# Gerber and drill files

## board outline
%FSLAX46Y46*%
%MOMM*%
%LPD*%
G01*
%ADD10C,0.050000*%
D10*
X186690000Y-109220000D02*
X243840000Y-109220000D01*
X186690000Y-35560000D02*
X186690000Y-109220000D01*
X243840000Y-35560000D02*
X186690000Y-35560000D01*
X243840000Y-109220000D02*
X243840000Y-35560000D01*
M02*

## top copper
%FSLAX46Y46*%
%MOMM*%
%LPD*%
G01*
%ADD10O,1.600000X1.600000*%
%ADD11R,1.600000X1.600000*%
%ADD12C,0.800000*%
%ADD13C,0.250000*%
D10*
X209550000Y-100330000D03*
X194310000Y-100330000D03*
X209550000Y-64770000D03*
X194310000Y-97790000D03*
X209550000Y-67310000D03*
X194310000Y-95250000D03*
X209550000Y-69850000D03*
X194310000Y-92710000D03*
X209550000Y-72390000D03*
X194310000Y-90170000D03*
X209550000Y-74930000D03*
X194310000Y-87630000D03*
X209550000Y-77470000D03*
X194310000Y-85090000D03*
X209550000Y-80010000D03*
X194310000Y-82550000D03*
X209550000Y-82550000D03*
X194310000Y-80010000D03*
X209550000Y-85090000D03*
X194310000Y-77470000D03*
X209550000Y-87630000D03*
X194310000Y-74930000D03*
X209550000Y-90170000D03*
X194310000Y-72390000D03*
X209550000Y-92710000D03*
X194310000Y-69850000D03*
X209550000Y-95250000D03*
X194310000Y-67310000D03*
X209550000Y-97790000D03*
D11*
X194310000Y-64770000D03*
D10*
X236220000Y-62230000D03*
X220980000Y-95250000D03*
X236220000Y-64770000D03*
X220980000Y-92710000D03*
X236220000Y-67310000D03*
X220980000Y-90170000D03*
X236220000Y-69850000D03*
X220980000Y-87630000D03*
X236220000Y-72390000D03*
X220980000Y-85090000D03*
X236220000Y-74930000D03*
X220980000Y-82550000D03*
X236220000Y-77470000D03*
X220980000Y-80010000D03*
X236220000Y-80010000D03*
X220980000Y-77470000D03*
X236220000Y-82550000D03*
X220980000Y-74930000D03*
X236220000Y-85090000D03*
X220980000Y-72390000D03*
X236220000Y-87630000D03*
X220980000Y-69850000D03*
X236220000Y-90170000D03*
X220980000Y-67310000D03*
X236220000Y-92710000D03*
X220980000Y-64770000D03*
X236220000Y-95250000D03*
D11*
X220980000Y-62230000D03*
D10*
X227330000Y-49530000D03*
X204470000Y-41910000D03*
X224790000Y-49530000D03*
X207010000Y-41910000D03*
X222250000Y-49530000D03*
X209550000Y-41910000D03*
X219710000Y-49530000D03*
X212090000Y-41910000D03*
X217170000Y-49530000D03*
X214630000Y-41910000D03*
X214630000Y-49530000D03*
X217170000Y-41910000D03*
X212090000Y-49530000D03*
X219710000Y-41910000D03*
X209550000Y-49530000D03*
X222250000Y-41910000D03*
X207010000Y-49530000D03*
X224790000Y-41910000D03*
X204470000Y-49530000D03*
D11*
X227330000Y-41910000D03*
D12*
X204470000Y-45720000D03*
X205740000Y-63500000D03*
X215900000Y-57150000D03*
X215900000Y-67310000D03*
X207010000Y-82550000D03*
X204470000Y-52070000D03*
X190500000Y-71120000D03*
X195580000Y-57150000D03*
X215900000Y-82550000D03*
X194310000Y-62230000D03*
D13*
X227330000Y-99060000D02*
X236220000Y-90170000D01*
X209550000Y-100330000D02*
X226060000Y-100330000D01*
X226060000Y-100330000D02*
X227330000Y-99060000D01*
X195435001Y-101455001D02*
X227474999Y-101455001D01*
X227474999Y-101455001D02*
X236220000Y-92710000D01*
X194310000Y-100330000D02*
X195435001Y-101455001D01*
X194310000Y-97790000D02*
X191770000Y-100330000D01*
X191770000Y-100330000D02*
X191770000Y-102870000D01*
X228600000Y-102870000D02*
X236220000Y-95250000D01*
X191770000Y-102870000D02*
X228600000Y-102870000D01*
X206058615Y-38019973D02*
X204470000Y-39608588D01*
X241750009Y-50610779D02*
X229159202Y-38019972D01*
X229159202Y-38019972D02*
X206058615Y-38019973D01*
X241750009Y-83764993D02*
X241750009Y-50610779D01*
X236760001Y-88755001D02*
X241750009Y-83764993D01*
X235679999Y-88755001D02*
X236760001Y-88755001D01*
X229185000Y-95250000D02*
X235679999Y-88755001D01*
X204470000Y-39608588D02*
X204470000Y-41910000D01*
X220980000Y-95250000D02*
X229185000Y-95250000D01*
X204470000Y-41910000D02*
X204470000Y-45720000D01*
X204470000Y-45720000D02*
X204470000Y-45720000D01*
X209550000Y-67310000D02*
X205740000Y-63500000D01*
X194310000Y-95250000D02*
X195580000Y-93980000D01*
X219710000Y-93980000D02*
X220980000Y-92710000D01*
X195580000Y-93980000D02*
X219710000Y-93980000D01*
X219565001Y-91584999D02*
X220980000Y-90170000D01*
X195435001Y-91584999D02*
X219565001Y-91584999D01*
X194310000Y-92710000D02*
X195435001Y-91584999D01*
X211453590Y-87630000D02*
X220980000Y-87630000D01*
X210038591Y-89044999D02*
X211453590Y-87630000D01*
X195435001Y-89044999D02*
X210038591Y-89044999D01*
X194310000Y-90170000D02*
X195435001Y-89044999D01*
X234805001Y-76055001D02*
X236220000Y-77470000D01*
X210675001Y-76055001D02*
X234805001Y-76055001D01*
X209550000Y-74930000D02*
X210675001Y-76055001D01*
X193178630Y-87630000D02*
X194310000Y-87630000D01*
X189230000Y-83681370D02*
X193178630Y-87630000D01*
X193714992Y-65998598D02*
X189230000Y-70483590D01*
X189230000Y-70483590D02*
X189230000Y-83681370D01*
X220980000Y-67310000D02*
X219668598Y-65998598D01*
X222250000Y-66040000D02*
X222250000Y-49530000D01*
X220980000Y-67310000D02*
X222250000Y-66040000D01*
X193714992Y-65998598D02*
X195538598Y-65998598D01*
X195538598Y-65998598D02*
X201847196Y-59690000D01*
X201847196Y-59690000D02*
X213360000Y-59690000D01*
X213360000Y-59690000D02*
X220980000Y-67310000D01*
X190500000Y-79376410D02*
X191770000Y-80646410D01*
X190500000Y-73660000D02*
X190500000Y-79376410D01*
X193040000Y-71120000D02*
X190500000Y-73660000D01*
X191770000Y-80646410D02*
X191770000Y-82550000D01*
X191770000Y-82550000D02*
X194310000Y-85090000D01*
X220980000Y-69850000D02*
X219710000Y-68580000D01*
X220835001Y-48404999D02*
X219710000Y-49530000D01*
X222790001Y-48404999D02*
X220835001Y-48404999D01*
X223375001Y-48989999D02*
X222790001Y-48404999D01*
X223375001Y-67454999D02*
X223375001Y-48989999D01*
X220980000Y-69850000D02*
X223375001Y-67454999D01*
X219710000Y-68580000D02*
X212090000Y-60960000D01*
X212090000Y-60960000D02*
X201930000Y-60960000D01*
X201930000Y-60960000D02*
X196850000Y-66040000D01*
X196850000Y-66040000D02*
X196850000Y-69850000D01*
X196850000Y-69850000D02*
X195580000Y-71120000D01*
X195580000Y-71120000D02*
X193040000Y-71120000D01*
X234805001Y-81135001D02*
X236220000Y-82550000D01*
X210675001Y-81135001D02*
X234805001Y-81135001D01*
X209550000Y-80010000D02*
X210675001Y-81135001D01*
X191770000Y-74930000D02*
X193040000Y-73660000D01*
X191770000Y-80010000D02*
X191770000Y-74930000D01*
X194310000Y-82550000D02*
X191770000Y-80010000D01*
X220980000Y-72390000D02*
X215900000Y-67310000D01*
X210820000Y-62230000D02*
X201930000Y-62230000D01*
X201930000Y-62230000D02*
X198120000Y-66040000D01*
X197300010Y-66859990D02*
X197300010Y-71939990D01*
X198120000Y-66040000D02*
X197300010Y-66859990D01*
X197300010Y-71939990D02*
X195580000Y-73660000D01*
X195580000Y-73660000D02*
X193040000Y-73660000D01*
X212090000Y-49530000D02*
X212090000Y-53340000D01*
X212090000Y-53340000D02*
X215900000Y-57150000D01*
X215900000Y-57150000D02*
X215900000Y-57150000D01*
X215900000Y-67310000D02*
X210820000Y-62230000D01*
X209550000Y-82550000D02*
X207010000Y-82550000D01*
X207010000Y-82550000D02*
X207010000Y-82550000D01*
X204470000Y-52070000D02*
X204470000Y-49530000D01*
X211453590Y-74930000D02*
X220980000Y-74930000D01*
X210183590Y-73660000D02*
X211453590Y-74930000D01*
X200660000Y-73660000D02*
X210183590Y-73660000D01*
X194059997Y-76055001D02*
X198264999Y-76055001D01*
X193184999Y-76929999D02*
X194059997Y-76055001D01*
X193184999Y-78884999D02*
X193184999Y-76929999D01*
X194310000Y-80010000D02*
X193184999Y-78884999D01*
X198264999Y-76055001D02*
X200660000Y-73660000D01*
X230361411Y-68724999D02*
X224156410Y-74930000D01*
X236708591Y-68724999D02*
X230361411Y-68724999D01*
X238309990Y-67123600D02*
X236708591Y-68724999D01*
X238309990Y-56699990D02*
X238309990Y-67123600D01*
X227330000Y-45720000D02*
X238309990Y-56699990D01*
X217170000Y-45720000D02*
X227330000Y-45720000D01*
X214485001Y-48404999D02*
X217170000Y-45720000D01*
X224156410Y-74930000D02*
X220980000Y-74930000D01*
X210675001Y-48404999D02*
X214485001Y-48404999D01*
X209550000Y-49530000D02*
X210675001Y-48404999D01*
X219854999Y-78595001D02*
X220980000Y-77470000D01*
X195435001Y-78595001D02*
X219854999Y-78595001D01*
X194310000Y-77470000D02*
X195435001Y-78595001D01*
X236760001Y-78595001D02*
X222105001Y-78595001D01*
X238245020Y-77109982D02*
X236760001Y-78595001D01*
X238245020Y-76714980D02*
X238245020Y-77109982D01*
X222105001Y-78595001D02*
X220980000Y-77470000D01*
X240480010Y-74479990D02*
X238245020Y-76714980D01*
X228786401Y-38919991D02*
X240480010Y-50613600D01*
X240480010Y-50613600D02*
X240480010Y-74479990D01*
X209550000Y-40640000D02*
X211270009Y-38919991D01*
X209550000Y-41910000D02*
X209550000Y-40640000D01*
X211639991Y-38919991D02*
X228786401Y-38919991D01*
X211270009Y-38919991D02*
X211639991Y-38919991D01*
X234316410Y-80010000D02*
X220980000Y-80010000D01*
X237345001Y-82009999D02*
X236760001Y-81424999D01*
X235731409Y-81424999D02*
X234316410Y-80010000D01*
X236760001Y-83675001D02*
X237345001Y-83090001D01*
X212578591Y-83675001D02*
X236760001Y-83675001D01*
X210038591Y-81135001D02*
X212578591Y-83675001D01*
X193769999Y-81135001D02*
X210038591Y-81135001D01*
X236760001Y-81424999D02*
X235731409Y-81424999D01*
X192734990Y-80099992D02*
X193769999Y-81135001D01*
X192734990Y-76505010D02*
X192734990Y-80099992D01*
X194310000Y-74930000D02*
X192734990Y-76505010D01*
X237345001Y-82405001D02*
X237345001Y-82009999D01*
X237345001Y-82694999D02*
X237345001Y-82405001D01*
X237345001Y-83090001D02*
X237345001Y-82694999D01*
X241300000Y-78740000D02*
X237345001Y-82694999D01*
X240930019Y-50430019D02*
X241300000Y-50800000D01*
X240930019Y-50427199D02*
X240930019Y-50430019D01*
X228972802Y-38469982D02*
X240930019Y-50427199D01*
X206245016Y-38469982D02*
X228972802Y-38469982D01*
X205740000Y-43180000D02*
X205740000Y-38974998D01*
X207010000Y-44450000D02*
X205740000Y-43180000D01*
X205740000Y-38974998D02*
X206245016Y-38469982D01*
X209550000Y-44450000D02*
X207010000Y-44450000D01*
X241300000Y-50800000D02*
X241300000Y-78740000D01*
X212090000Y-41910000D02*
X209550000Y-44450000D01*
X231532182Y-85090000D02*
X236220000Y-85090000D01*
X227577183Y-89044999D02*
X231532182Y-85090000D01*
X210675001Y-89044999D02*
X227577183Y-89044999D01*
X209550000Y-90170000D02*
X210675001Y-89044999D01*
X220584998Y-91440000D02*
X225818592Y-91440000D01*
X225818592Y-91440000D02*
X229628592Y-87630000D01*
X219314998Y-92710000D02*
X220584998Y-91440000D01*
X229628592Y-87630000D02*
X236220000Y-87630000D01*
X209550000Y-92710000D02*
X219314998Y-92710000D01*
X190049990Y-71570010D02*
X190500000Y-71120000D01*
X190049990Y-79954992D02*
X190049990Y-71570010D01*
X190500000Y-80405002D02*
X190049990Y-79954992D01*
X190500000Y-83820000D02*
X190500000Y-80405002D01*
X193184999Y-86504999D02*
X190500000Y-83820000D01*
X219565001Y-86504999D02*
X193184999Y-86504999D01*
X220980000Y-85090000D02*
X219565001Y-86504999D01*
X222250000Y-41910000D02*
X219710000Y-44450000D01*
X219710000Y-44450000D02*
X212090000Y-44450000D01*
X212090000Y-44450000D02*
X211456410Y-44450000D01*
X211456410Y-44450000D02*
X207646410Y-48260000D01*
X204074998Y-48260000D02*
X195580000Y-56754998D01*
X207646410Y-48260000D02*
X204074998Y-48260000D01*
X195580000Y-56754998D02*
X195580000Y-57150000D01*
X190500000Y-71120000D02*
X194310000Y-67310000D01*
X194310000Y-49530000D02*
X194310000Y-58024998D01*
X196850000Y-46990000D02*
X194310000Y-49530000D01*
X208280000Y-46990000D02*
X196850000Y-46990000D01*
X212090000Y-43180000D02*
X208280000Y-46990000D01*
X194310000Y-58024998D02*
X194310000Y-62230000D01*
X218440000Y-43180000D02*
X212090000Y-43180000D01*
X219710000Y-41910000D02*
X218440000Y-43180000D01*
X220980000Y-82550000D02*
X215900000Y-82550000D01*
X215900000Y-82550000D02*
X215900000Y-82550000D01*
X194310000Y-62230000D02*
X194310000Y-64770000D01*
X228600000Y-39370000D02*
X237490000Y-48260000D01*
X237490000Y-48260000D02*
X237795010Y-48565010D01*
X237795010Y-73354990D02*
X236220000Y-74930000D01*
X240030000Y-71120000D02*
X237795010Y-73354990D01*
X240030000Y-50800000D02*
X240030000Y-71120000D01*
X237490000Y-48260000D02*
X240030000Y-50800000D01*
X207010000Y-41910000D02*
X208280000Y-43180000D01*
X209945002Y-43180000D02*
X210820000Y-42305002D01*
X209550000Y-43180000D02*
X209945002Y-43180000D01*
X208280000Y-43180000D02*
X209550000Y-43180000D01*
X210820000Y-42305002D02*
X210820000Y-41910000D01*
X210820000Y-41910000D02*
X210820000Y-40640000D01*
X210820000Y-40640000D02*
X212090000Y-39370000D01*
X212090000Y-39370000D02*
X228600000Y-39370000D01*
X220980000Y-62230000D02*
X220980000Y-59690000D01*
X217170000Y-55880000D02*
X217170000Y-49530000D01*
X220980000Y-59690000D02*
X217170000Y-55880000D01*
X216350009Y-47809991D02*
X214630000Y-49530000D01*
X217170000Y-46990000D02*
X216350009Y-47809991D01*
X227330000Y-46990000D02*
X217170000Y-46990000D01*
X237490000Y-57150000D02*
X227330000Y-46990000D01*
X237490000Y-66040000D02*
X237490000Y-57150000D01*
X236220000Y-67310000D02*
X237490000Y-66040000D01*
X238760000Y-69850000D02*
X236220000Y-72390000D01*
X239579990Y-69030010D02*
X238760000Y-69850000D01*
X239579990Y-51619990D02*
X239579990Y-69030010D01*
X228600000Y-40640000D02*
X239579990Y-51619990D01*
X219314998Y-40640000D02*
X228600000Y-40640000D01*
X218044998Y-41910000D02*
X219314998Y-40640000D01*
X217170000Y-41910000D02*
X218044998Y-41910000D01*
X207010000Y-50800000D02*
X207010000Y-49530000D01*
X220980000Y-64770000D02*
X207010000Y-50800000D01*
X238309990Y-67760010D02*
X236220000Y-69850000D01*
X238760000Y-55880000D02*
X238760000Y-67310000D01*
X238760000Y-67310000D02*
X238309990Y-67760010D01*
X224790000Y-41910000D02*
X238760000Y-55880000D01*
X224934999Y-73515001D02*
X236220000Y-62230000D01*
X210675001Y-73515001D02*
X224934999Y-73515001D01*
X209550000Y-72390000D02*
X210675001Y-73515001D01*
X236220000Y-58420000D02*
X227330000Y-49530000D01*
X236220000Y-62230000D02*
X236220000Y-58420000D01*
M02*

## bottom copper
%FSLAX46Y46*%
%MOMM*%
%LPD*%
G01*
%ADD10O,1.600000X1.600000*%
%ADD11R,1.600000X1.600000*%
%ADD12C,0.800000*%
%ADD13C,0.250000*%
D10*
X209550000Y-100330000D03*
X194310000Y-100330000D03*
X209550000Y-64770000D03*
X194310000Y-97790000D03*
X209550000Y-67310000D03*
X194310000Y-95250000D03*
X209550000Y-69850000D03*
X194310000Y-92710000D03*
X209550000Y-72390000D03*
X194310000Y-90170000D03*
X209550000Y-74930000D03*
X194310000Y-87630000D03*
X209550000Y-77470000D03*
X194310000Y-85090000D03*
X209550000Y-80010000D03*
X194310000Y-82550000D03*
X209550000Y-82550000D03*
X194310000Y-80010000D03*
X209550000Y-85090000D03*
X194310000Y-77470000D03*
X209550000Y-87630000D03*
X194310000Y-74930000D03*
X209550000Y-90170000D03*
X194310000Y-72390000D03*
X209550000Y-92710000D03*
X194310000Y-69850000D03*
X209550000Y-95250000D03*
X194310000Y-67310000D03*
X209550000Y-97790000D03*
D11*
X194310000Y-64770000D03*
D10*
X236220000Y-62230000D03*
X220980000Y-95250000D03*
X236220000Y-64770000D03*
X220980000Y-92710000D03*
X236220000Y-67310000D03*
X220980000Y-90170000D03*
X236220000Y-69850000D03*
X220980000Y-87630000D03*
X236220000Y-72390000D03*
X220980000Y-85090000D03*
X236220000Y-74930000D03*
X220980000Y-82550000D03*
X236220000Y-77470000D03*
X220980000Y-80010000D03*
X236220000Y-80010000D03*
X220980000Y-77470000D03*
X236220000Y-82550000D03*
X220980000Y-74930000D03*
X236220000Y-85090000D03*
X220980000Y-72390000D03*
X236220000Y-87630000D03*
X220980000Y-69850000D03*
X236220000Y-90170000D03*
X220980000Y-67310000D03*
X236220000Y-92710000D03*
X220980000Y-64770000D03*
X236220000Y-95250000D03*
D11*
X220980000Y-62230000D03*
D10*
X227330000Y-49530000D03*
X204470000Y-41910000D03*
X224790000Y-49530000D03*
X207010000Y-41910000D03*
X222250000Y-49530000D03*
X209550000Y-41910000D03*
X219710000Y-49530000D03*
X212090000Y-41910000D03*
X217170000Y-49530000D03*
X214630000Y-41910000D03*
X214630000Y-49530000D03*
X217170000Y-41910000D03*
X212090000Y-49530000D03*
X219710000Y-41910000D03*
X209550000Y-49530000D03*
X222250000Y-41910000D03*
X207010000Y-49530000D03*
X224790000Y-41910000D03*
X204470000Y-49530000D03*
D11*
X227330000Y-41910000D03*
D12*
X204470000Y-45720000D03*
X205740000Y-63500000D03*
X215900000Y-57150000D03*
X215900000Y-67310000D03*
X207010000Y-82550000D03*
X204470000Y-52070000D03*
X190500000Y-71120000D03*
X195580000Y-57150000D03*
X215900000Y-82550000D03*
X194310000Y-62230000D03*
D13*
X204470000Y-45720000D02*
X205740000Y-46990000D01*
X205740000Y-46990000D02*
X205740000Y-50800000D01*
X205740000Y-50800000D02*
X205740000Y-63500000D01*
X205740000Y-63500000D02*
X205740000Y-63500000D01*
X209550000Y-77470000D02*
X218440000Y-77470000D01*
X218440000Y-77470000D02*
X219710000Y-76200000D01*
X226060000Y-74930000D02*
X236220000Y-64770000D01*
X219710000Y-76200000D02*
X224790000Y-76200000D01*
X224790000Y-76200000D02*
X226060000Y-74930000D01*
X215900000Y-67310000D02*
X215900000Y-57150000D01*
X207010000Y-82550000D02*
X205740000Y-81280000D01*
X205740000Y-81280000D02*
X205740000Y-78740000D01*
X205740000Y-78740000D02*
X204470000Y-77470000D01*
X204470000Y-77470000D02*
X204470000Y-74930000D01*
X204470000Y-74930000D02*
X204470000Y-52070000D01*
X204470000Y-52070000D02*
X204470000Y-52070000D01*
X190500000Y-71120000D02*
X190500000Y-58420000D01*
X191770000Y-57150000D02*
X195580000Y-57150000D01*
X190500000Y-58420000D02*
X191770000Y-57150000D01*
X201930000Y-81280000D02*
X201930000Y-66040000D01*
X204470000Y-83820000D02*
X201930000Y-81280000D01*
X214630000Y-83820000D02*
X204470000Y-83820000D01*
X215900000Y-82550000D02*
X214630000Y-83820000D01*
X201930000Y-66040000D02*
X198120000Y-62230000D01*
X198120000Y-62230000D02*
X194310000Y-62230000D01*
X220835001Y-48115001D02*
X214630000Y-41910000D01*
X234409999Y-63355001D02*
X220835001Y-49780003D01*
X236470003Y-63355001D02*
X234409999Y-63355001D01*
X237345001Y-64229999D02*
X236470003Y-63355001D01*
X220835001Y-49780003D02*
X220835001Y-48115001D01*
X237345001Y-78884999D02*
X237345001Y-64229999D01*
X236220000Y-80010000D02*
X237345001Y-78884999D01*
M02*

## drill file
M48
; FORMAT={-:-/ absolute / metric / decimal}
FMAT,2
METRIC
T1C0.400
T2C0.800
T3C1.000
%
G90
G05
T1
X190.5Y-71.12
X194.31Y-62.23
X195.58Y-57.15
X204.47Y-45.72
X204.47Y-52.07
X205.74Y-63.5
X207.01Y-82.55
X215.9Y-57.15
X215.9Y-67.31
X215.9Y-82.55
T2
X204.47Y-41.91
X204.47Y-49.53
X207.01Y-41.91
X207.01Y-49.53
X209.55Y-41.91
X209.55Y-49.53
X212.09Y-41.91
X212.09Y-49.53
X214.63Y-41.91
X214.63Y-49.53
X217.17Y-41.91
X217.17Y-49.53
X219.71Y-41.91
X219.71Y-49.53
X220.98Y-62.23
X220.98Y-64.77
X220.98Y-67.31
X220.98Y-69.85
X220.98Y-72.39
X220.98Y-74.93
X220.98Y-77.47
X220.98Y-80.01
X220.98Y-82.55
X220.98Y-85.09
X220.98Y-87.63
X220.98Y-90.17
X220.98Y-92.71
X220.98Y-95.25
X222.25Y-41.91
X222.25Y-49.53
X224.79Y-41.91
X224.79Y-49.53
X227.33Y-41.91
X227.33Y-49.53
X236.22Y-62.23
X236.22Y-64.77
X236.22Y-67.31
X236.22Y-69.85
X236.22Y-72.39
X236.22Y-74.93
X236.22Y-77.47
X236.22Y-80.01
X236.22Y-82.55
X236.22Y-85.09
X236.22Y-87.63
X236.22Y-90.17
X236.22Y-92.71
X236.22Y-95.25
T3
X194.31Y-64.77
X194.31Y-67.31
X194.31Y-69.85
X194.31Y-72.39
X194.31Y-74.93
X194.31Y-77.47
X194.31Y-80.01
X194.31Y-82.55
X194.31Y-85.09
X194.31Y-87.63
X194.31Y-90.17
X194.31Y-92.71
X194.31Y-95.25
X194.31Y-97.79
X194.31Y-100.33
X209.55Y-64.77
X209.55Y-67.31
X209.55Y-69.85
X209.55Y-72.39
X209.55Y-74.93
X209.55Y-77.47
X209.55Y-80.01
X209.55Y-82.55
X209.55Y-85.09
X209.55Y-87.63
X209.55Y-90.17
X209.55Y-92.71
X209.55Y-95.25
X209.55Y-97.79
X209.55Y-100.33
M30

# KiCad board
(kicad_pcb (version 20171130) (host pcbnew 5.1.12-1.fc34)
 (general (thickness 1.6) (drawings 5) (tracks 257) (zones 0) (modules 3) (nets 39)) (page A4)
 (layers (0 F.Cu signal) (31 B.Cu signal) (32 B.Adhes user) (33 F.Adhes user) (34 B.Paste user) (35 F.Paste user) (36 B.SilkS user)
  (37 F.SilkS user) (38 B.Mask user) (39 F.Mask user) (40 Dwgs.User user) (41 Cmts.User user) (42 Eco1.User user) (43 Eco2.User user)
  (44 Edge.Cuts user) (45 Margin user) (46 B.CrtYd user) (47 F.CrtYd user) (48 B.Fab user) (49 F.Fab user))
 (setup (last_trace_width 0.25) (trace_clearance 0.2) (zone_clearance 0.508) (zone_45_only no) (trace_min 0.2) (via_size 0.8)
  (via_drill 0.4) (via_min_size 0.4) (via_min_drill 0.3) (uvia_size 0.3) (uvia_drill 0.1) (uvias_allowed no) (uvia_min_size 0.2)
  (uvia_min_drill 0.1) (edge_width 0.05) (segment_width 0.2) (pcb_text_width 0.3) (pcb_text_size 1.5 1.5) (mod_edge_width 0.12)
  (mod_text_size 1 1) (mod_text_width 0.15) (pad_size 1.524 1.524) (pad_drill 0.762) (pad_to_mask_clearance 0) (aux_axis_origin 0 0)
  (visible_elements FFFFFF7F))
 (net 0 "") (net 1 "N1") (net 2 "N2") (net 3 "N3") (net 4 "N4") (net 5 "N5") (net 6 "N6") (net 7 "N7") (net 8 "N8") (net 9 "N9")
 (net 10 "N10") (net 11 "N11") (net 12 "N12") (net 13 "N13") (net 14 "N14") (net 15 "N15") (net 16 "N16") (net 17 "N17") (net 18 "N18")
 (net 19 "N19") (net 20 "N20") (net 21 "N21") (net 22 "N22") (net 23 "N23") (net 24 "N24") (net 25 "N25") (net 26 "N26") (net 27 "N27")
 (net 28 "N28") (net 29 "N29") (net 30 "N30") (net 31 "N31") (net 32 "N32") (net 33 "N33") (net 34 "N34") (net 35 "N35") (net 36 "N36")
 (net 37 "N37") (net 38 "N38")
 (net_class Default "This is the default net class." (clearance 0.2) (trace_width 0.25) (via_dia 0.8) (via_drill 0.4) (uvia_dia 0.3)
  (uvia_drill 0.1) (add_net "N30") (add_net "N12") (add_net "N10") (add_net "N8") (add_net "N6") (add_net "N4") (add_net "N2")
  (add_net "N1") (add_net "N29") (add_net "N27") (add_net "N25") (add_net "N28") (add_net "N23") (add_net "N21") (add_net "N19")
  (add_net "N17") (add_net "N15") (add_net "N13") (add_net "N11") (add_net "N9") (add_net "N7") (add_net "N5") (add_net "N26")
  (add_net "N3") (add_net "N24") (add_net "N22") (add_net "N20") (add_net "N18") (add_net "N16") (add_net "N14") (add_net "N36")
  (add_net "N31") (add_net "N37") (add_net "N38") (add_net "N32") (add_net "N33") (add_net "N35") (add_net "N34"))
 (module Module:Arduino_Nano (layer F.Cu) (at 194.31 64.77)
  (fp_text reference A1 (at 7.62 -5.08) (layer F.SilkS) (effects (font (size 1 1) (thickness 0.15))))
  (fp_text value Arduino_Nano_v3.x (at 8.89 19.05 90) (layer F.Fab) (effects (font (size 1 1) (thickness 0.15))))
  (pad 16 thru_hole oval (at 15.24 35.56) (size 1.6 1.6) (drill 1) (layers *.Cu *.Mask) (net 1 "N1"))
  (pad 15 thru_hole oval (at 0 35.56) (size 1.6 1.6) (drill 1) (layers *.Cu *.Mask) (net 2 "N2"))
  (pad 30 thru_hole oval (at 15.24 0) (size 1.6 1.6) (drill 1) (layers *.Cu *.Mask) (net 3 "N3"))
  (pad 14 thru_hole oval (at 0 33.02) (size 1.6 1.6) (drill 1) (layers *.Cu *.Mask) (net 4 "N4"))
  (pad 29 thru_hole oval (at 15.24 2.54) (size 1.6 1.6) (drill 1) (layers *.Cu *.Mask) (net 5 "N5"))
  (pad 13 thru_hole oval (at 0 30.48) (size 1.6 1.6) (drill 1) (layers *.Cu *.Mask) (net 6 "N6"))
  (pad 28 thru_hole oval (at 15.24 5.08) (size 1.6 1.6) (drill 1) (layers *.Cu *.Mask) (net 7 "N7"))
  (pad 12 thru_hole oval (at 0 27.94) (size 1.6 1.6) (drill 1) (layers *.Cu *.Mask) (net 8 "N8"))
  (pad 27 thru_hole oval (at 15.24 7.62) (size 1.6 1.6) (drill 1) (layers *.Cu *.Mask) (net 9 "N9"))
  (pad 11 thru_hole oval (at 0 25.4) (size 1.6 1.6) (drill 1) (layers *.Cu *.Mask) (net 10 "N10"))
  (pad 26 thru_hole oval (at 15.24 10.16) (size 1.6 1.6) (drill 1) (layers *.Cu *.Mask) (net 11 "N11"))
  (pad 10 thru_hole oval (at 0 22.86) (size 1.6 1.6) (drill 1) (layers *.Cu *.Mask) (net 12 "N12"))
  (pad 25 thru_hole oval (at 15.24 12.7) (size 1.6 1.6) (drill 1) (layers *.Cu *.Mask) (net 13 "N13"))
  (pad 9 thru_hole oval (at 0 20.32) (size 1.6 1.6) (drill 1) (layers *.Cu *.Mask) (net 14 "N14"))
  (pad 24 thru_hole oval (at 15.24 15.24) (size 1.6 1.6) (drill 1) (layers *.Cu *.Mask) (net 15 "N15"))
  (pad 8 thru_hole oval (at 0 17.78) (size 1.6 1.6) (drill 1) (layers *.Cu *.Mask) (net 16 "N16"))
  (pad 23 thru_hole oval (at 15.24 17.78) (size 1.6 1.6) (drill 1) (layers *.Cu *.Mask) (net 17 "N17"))
  (pad 7 thru_hole oval (at 0 15.24) (size 1.6 1.6) (drill 1) (layers *.Cu *.Mask) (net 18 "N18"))
  (pad 22 thru_hole oval (at 15.24 20.32) (size 1.6 1.6) (drill 1) (layers *.Cu *.Mask) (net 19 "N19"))
  (pad 6 thru_hole oval (at 0 12.7) (size 1.6 1.6) (drill 1) (layers *.Cu *.Mask) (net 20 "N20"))
  (pad 21 thru_hole oval (at 15.24 22.86) (size 1.6 1.6) (drill 1) (layers *.Cu *.Mask) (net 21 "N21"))
  (pad 5 thru_hole oval (at 0 10.16) (size 1.6 1.6) (drill 1) (layers *.Cu *.Mask) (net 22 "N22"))
  (pad 20 thru_hole oval (at 15.24 25.4) (size 1.6 1.6) (drill 1) (layers *.Cu *.Mask) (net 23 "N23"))
  (pad 4 thru_hole oval (at 0 7.62) (size 1.6 1.6) (drill 1) (layers *.Cu *.Mask) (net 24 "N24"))
  (pad 19 thru_hole oval (at 15.24 27.94) (size 1.6 1.6) (drill 1) (layers *.Cu *.Mask) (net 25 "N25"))
  (pad 3 thru_hole oval (at 0 5.08) (size 1.6 1.6) (drill 1) (layers *.Cu *.Mask) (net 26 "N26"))
  (pad 18 thru_hole oval (at 15.24 30.48) (size 1.6 1.6) (drill 1) (layers *.Cu *.Mask) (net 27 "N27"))
  (pad 2 thru_hole oval (at 0 2.54) (size 1.6 1.6) (drill 1) (layers *.Cu *.Mask) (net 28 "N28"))
  (pad 17 thru_hole oval (at 15.24 33.02) (size 1.6 1.6) (drill 1) (layers *.Cu *.Mask) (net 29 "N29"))
  (pad 1 thru_hole rect (at 0 0) (size 1.6 1.6) (drill 1) (layers *.Cu *.Mask) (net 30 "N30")))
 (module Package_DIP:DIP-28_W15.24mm (layer F.Cu) (at 220.98 62.23)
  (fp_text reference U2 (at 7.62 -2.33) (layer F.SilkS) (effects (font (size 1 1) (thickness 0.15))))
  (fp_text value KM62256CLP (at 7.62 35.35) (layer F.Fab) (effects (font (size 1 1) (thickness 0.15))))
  (pad 28 thru_hole oval (at 15.24 0) (size 1.6 1.6) (drill 0.8) (layers *.Cu *.Mask) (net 9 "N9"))
  (pad 14 thru_hole oval (at 0 33.02) (size 1.6 1.6) (drill 0.8) (layers *.Cu *.Mask) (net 5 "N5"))
  (pad 27 thru_hole oval (at 15.24 2.54) (size 1.6 1.6) (drill 0.8) (layers *.Cu *.Mask) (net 13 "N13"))
  (pad 13 thru_hole oval (at 0 30.48) (size 1.6 1.6) (drill 0.8) (layers *.Cu *.Mask) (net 6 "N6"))
  (pad 26 thru_hole oval (at 15.24 5.08) (size 1.6 1.6) (drill 0.8) (layers *.Cu *.Mask) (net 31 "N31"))
  (pad 12 thru_hole oval (at 0 27.94) (size 1.6 1.6) (drill 0.8) (layers *.Cu *.Mask) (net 8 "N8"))
  (pad 25 thru_hole oval (at 15.24 7.62) (size 1.6 1.6) (drill 0.8) (layers *.Cu *.Mask) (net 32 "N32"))
  (pad 11 thru_hole oval (at 0 25.4) (size 1.6 1.6) (drill 0.8) (layers *.Cu *.Mask) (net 10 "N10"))
  (pad 24 thru_hole oval (at 15.24 10.16) (size 1.6 1.6) (drill 0.8) (layers *.Cu *.Mask) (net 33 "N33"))
  (pad 10 thru_hole oval (at 0 22.86) (size 1.6 1.6) (drill 0.8) (layers *.Cu *.Mask) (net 28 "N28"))
  (pad 23 thru_hole oval (at 15.24 12.7) (size 1.6 1.6) (drill 0.8) (layers *.Cu *.Mask) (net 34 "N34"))
  (pad 9 thru_hole oval (at 0 20.32) (size 1.6 1.6) (drill 0.8) (layers *.Cu *.Mask) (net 30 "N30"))
  (pad 22 thru_hole oval (at 15.24 15.24) (size 1.6 1.6) (drill 0.8) (layers *.Cu *.Mask) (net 11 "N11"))
  (pad 8 thru_hole oval (at 0 17.78) (size 1.6 1.6) (drill 0.8) (layers *.Cu *.Mask) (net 22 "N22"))
  (pad 21 thru_hole oval (at 15.24 17.78) (size 1.6 1.6) (drill 0.8) (layers *.Cu *.Mask) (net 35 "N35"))
  (pad 7 thru_hole oval (at 0 15.24) (size 1.6 1.6) (drill 0.8) (layers *.Cu *.Mask) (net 20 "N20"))
  (pad 20 thru_hole oval (at 15.24 20.32) (size 1.6 1.6) (drill 0.8) (layers *.Cu *.Mask) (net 15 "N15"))
  (pad 6 thru_hole oval (at 0 12.7) (size 1.6 1.6) (drill 0.8) (layers *.Cu *.Mask) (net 18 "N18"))
  (pad 19 thru_hole oval (at 15.24 22.86) (size 1.6 1.6) (drill 0.8) (layers *.Cu *.Mask) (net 23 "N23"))
  (pad 5 thru_hole oval (at 0 10.16) (size 1.6 1.6) (drill 0.8) (layers *.Cu *.Mask) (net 16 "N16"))
  (pad 18 thru_hole oval (at 15.24 25.4) (size 1.6 1.6) (drill 0.8) (layers *.Cu *.Mask) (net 25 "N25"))
  (pad 4 thru_hole oval (at 0 7.62) (size 1.6 1.6) (drill 0.8) (layers *.Cu *.Mask) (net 14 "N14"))
  (pad 17 thru_hole oval (at 15.24 27.94) (size 1.6 1.6) (drill 0.8) (layers *.Cu *.Mask) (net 1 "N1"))
  (pad 3 thru_hole oval (at 0 5.08) (size 1.6 1.6) (drill 0.8) (layers *.Cu *.Mask) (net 12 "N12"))
  (pad 16 thru_hole oval (at 15.24 30.48) (size 1.6 1.6) (drill 0.8) (layers *.Cu *.Mask) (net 2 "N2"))
  (pad 2 thru_hole oval (at 0 2.54) (size 1.6 1.6) (drill 0.8) (layers *.Cu *.Mask) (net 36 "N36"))
  (pad 15 thru_hole oval (at 15.24 33.02) (size 1.6 1.6) (drill 0.8) (layers *.Cu *.Mask) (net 4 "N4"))
  (pad 1 thru_hole rect (at 0 0) (size 1.6 1.6) (drill 0.8) (layers *.Cu *.Mask) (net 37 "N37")))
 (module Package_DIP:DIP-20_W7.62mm (layer F.Cu) (at 227.33 41.91 270)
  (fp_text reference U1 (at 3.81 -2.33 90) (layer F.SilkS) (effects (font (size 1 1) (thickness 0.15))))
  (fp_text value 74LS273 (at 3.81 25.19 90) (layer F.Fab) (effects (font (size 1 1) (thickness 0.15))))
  (pad 20 thru_hole oval (at 7.62 0 270) (size 1.6 1.6) (drill 0.8) (layers *.Cu *.Mask) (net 9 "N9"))
  (pad 10 thru_hole oval (at 0 22.86 270) (size 1.6 1.6) (drill 0.8) (layers *.Cu *.Mask) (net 5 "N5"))
  (pad 19 thru_hole oval (at 7.62 2.54 270) (size 1.6 1.6) (drill 0.8) (layers *.Cu *.Mask) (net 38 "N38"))
  (pad 9 thru_hole oval (at 0 20.32 270) (size 1.6 1.6) (drill 0.8) (layers *.Cu *.Mask) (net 34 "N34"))
  (pad 18 thru_hole oval (at 7.62 5.08 270) (size 1.6 1.6) (drill 0.8) (layers *.Cu *.Mask) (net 12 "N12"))
  (pad 8 thru_hole oval (at 0 17.78 270) (size 1.6 1.6) (drill 0.8) (layers *.Cu *.Mask) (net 20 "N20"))
  (pad 17 thru_hole oval (at 7.62 7.62 270) (size 1.6 1.6) (drill 0.8) (layers *.Cu *.Mask) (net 14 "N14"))
  (pad 7 thru_hole oval (at 0 15.24 270) (size 1.6 1.6) (drill 0.8) (layers *.Cu *.Mask) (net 22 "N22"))
  (pad 16 thru_hole oval (at 7.62 10.16 270) (size 1.6 1.6) (drill 0.8) (layers *.Cu *.Mask) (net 37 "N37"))
  (pad 6 thru_hole oval (at 0 12.7 270) (size 1.6 1.6) (drill 0.8) (layers *.Cu *.Mask) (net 35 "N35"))
  (pad 15 thru_hole oval (at 7.62 12.7 270) (size 1.6 1.6) (drill 0.8) (layers *.Cu *.Mask) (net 31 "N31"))
  (pad 5 thru_hole oval (at 0 10.16 270) (size 1.6 1.6) (drill 0.8) (layers *.Cu *.Mask) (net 33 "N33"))
  (pad 14 thru_hole oval (at 7.62 15.24 270) (size 1.6 1.6) (drill 0.8) (layers *.Cu *.Mask) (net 16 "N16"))
  (pad 4 thru_hole oval (at 0 7.62 270) (size 1.6 1.6) (drill 0.8) (layers *.Cu *.Mask) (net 30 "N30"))
  (pad 13 thru_hole oval (at 7.62 17.78 270) (size 1.6 1.6) (drill 0.8) (layers *.Cu *.Mask) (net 18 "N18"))
  (pad 3 thru_hole oval (at 0 5.08 270) (size 1.6 1.6) (drill 0.8) (layers *.Cu *.Mask) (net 28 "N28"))
  (pad 12 thru_hole oval (at 7.62 20.32 270) (size 1.6 1.6) (drill 0.8) (layers *.Cu *.Mask) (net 36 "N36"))
  (pad 2 thru_hole oval (at 0 2.54 270) (size 1.6 1.6) (drill 0.8) (layers *.Cu *.Mask) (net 32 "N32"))
  (pad 11 thru_hole oval (at 7.62 22.86 270) (size 1.6 1.6) (drill 0.8) (layers *.Cu *.Mask) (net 17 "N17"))
  (pad 1 thru_hole rect (at 0 0 270) (size 1.6 1.6) (drill 0.8) (layers *.Cu *.Mask) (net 9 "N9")))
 (gr_line (start 186.69 109.22) (end 243.84 109.22) (layer Edge.Cuts) (width 0.05))
 (gr_line (start 186.69 35.56) (end 186.69 109.22) (layer Edge.Cuts) (width 0.05))
 (gr_line (start 243.84 35.56) (end 186.69 35.56) (layer Edge.Cuts) (width 0.05))
 (gr_line (start 243.84 109.22) (end 243.84 35.56) (layer Edge.Cuts) (width 0.05))
 (segment (start 227.33 99.06) (end 236.22 90.17) (width 0.25) (layer F.Cu) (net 1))
 (segment (start 209.55 100.33) (end 226.06 100.33) (width 0.25) (layer F.Cu) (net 1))
 (segment (start 226.06 100.33) (end 227.33 99.06) (width 0.25) (layer F.Cu) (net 1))
 (segment (start 195.435001 101.455001) (end 227.474999 101.455001) (width 0.25) (layer F.Cu) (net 2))
 (segment (start 227.474999 101.455001) (end 236.22 92.71) (width 0.25) (layer F.Cu) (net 2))
 (segment (start 194.31 100.33) (end 195.435001 101.455001) (width 0.25) (layer F.Cu) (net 2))
 (segment (start 194.31 97.79) (end 191.77 100.33) (width 0.25) (layer F.Cu) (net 4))
 (segment (start 191.77 100.33) (end 191.77 102.87) (width 0.25) (layer F.Cu) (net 4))
 (segment (start 228.6 102.87) (end 236.22 95.25) (width 0.25) (layer F.Cu) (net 4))
 (segment (start 191.77 102.87) (end 228.6 102.87) (width 0.25) (layer F.Cu) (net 4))
 (segment (start 206.058615 38.019973) (end 204.47 39.608588) (width 0.25) (layer F.Cu) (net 5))
 (segment (start 241.750009 50.610779) (end 229.159202 38.019972) (width 0.25) (layer F.Cu) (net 5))
 (segment (start 229.159202 38.019972) (end 206.058615 38.019973) (width 0.25) (layer F.Cu) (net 5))
 (segment (start 241.750009 83.764993) (end 241.750009 50.610779) (width 0.25) (layer F.Cu) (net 5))
 (segment (start 236.760001 88.755001) (end 241.750009 83.764993) (width 0.25) (layer F.Cu) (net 5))
 (segment (start 235.679999 88.755001) (end 236.760001 88.755001) (width 0.25) (layer F.Cu) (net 5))
 (segment (start 229.185 95.25) (end 235.679999 88.755001) (width 0.25) (layer F.Cu) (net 5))
 (segment (start 204.47 39.608588) (end 204.47 41.91) (width 0.25) (layer F.Cu) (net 5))
 (segment (start 220.98 95.25) (end 229.185 95.25) (width 0.25) (layer F.Cu) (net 5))
 (segment (start 204.47 41.91) (end 204.47 45.72) (width 0.25) (layer F.Cu) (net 5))
 (segment (start 204.47 45.72) (end 204.47 45.72) (width 0.25) (layer F.Cu) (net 5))
 (via (at 204.47 45.72) (size 0.8) (drill 0.4) (layers F.Cu B.Cu) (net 5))
 (segment (start 204.47 45.72) (end 205.74 46.99) (width 0.25) (layer B.Cu) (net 5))
 (segment (start 205.74 46.99) (end 205.74 50.8) (width 0.25) (layer B.Cu) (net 5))
 (segment (start 205.74 50.8) (end 205.74 63.5) (width 0.25) (layer B.Cu) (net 5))
 (segment (start 205.74 63.5) (end 205.74 63.5) (width 0.25) (layer B.Cu) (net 5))
 (via (at 205.74 63.5) (size 0.8) (drill 0.4) (layers F.Cu B.Cu) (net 5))
 (segment (start 209.55 67.31) (end 205.74 63.5) (width 0.25) (layer F.Cu) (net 5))
 (segment (start 194.31 95.25) (end 195.58 93.98) (width 0.25) (layer F.Cu) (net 6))
 (segment (start 219.71 93.98) (end 220.98 92.71) (width 0.25) (layer F.Cu) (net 6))
 (segment (start 195.58 93.98) (end 219.71 93.98) (width 0.25) (layer F.Cu) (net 6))
 (segment (start 219.565001 91.584999) (end 220.98 90.17) (width 0.25) (layer F.Cu) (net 8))
 (segment (start 195.435001 91.584999) (end 219.565001 91.584999) (width 0.25) (layer F.Cu) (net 8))
 (segment (start 194.31 92.71) (end 195.435001 91.584999) (width 0.25) (layer F.Cu) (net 8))
 (segment (start 211.45359 87.63) (end 220.98 87.63) (width 0.25) (layer F.Cu) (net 10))
 (segment (start 210.038591 89.044999) (end 211.45359 87.63) (width 0.25) (layer F.Cu) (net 10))
 (segment (start 195.435001 89.044999) (end 210.038591 89.044999) (width 0.25) (layer F.Cu) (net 10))
 (segment (start 194.31 90.17) (end 195.435001 89.044999) (width 0.25) (layer F.Cu) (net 10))
 (segment (start 234.805001 76.055001) (end 236.22 77.47) (width 0.25) (layer F.Cu) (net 11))
 (segment (start 210.675001 76.055001) (end 234.805001 76.055001) (width 0.25) (layer F.Cu) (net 11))
 (segment (start 209.55 74.93) (end 210.675001 76.055001) (width 0.25) (layer F.Cu) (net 11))
 (segment (start 193.17863 87.63) (end 194.31 87.63) (width 0.25) (layer F.Cu) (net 12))
 (segment (start 189.23 83.68137) (end 193.17863 87.63) (width 0.25) (layer F.Cu) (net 12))
 (segment (start 193.714992 65.998598) (end 189.23 70.48359) (width 0.25) (layer F.Cu) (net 12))
 (segment (start 189.23 70.48359) (end 189.23 83.68137) (width 0.25) (layer F.Cu) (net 12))
 (segment (start 220.98 67.31) (end 219.668598 65.998598) (width 0.25) (layer F.Cu) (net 12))
 (segment (start 222.25 66.04) (end 222.25 49.53) (width 0.25) (layer F.Cu) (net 12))
 (segment (start 220.98 67.31) (end 222.25 66.04) (width 0.25) (layer F.Cu) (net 12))
 (segment (start 193.714992 65.998598) (end 195.538598 65.998598) (width 0.25) (layer F.Cu) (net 12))
 (segment (start 195.538598 65.998598) (end 201.847196 59.69) (width 0.25) (layer F.Cu) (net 12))
 (segment (start 201.847196 59.69) (end 213.36 59.69) (width 0.25) (layer F.Cu) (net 12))
 (segment (start 213.36 59.69) (end 220.98 67.31) (width 0.25) (layer F.Cu) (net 12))
 (segment (start 209.55 77.47) (end 218.44 77.47) (width 0.25) (layer B.Cu) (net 13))
 (segment (start 218.44 77.47) (end 219.71 76.2) (width 0.25) (layer B.Cu) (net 13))
 (segment (start 226.06 74.93) (end 236.22 64.77) (width 0.25) (layer B.Cu) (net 13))
 (segment (start 219.71 76.2) (end 224.79 76.2) (width 0.25) (layer B.Cu) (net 13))
 (segment (start 224.79 76.2) (end 226.06 74.93) (width 0.25) (layer B.Cu) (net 13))
 (segment (start 190.5 79.37641) (end 191.77 80.64641) (width 0.25) (layer F.Cu) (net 14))
 (segment (start 190.5 73.66) (end 190.5 79.37641) (width 0.25) (layer F.Cu) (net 14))
 (segment (start 193.04 71.12) (end 190.5 73.66) (width 0.25) (layer F.Cu) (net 14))
 (segment (start 191.77 80.64641) (end 191.77 82.55) (width 0.25) (layer F.Cu) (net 14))
 (segment (start 191.77 82.55) (end 194.31 85.09) (width 0.25) (layer F.Cu) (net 14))
 (segment (start 220.98 69.85) (end 219.71 68.58) (width 0.25) (layer F.Cu) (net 14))
 (segment (start 220.835001 48.404999) (end 219.71 49.53) (width 0.25) (layer F.Cu) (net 14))
 (segment (start 222.790001 48.404999) (end 220.835001 48.404999) (width 0.25) (layer F.Cu) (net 14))
 (segment (start 223.375001 48.989999) (end 222.790001 48.404999) (width 0.25) (layer F.Cu) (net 14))
 (segment (start 223.375001 67.454999) (end 223.375001 48.989999) (width 0.25) (layer F.Cu) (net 14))
 (segment (start 220.98 69.85) (end 223.375001 67.454999) (width 0.25) (layer F.Cu) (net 14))
 (segment (start 219.71 68.58) (end 212.09 60.96) (width 0.25) (layer F.Cu) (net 14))
 (segment (start 212.09 60.96) (end 201.93 60.96) (width 0.25) (layer F.Cu) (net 14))
 (segment (start 201.93 60.96) (end 196.85 66.04) (width 0.25) (layer F.Cu) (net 14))
 (segment (start 196.85 66.04) (end 196.85 69.85) (width 0.25) (layer F.Cu) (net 14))
 (segment (start 196.85 69.85) (end 195.58 71.12) (width 0.25) (layer F.Cu) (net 14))
 (segment (start 195.58 71.12) (end 193.04 71.12) (width 0.25) (layer F.Cu) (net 14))
 (segment (start 234.805001 81.135001) (end 236.22 82.55) (width 0.25) (layer F.Cu) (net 15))
 (segment (start 210.675001 81.135001) (end 234.805001 81.135001) (width 0.25) (layer F.Cu) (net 15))
 (segment (start 209.55 80.01) (end 210.675001 81.135001) (width 0.25) (layer F.Cu) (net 15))
 (segment (start 191.77 74.93) (end 193.04 73.66) (width 0.25) (layer F.Cu) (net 16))
 (segment (start 191.77 80.01) (end 191.77 74.93) (width 0.25) (layer F.Cu) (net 16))
 (segment (start 194.31 82.55) (end 191.77 80.01) (width 0.25) (layer F.Cu) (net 16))
 (segment (start 220.98 72.39) (end 215.9 67.31) (width 0.25) (layer F.Cu) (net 16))
 (segment (start 210.82 62.23) (end 201.93 62.23) (width 0.25) (layer F.Cu) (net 16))
 (segment (start 201.93 62.23) (end 198.12 66.04) (width 0.25) (layer F.Cu) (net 16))
 (segment (start 197.30001 66.85999) (end 197.30001 71.93999) (width 0.25) (layer F.Cu) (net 16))
 (segment (start 198.12 66.04) (end 197.30001 66.85999) (width 0.25) (layer F.Cu) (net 16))
 (segment (start 197.30001 71.93999) (end 195.58 73.66) (width 0.25) (layer F.Cu) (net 16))
 (segment (start 195.58 73.66) (end 193.04 73.66) (width 0.25) (layer F.Cu) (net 16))
 (segment (start 212.09 49.53) (end 212.09 53.34) (width 0.25) (layer F.Cu) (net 16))
 (segment (start 212.09 53.34) (end 215.9 57.15) (width 0.25) (layer F.Cu) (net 16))
 (segment (start 215.9 57.15) (end 215.9 57.15) (width 0.25) (layer F.Cu) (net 16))
 (via (at 215.9 57.15) (size 0.8) (drill 0.4) (layers F.Cu B.Cu) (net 16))
 (segment (start 215.9 67.31) (end 210.82 62.23) (width 0.25) (layer F.Cu) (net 16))
 (via (at 215.9 67.31) (size 0.8) (drill 0.4) (layers F.Cu B.Cu) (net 16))
 (segment (start 215.9 67.31) (end 215.9 57.15) (width 0.25) (layer B.Cu) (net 16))
 (segment (start 209.55 82.55) (end 207.01 82.55) (width 0.25) (layer F.Cu) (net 17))
 (segment (start 207.01 82.55) (end 207.01 82.55) (width 0.25) (layer F.Cu) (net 17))
 (via (at 207.01 82.55) (size 0.8) (drill 0.4) (layers F.Cu B.Cu) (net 17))
 (segment (start 207.01 82.55) (end 205.74 81.28) (width 0.25) (layer B.Cu) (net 17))
 (segment (start 205.74 81.28) (end 205.74 78.74) (width 0.25) (layer B.Cu) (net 17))
 (segment (start 205.74 78.74) (end 204.47 77.47) (width 0.25) (layer B.Cu) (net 17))
 (segment (start 204.47 77.47) (end 204.47 74.93) (width 0.25) (layer B.Cu) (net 17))
 (segment (start 204.47 74.93) (end 204.47 52.07) (width 0.25) (layer B.Cu) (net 17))
 (segment (start 204.47 52.07) (end 204.47 52.07) (width 0.25) (layer B.Cu) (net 17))
 (via (at 204.47 52.07) (size 0.8) (drill 0.4) (layers F.Cu B.Cu) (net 17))
 (segment (start 204.47 52.07) (end 204.47 49.53) (width 0.25) (layer F.Cu) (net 17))
 (segment (start 211.45359 74.93) (end 220.98 74.93) (width 0.25) (layer F.Cu) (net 18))
 (segment (start 210.18359 73.66) (end 211.45359 74.93) (width 0.25) (layer F.Cu) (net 18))
 (segment (start 200.66 73.66) (end 210.18359 73.66) (width 0.25) (layer F.Cu) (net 18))
 (segment (start 194.059997 76.055001) (end 198.264999 76.055001) (width 0.25) (layer F.Cu) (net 18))
 (segment (start 193.184999 76.929999) (end 194.059997 76.055001) (width 0.25) (layer F.Cu) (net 18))
 (segment (start 193.184999 78.884999) (end 193.184999 76.929999) (width 0.25) (layer F.Cu) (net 18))
 (segment (start 194.31 80.01) (end 193.184999 78.884999) (width 0.25) (layer F.Cu) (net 18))
 (segment (start 198.264999 76.055001) (end 200.66 73.66) (width 0.25) (layer F.Cu) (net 18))
 (segment (start 230.361411 68.724999) (end 224.15641 74.93) (width 0.25) (layer F.Cu) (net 18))
 (segment (start 236.708591 68.724999) (end 230.361411 68.724999) (width 0.25) (layer F.Cu) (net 18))
 (segment (start 238.30999 67.1236) (end 236.708591 68.724999) (width 0.25) (layer F.Cu) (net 18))
 (segment (start 238.30999 56.69999) (end 238.30999 67.1236) (width 0.25) (layer F.Cu) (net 18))
 (segment (start 227.33 45.72) (end 238.30999 56.69999) (width 0.25) (layer F.Cu) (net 18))
 (segment (start 217.17 45.72) (end 227.33 45.72) (width 0.25) (layer F.Cu) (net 18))
 (segment (start 214.485001 48.404999) (end 217.17 45.72) (width 0.25) (layer F.Cu) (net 18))
 (segment (start 224.15641 74.93) (end 220.98 74.93) (width 0.25) (layer F.Cu) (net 18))
 (segment (start 210.675001 48.404999) (end 214.485001 48.404999) (width 0.25) (layer F.Cu) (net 18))
 (segment (start 209.55 49.53) (end 210.675001 48.404999) (width 0.25) (layer F.Cu) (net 18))
 (segment (start 219.854999 78.595001) (end 220.98 77.47) (width 0.25) (layer F.Cu) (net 20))
 (segment (start 195.435001 78.595001) (end 219.854999 78.595001) (width 0.25) (layer F.Cu) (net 20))
 (segment (start 194.31 77.47) (end 195.435001 78.595001) (width 0.25) (layer F.Cu) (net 20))
 (segment (start 236.760001 78.595001) (end 222.105001 78.595001) (width 0.25) (layer F.Cu) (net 20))
 (segment (start 238.24502 77.109982) (end 236.760001 78.595001) (width 0.25) (layer F.Cu) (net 20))
 (segment (start 238.24502 76.71498) (end 238.24502 77.109982) (width 0.25) (layer F.Cu) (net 20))
 (segment (start 222.105001 78.595001) (end 220.98 77.47) (width 0.25) (layer F.Cu) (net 20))
 (segment (start 240.48001 74.47999) (end 238.24502 76.71498) (width 0.25) (layer F.Cu) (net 20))
 (segment (start 228.786401 38.919991) (end 240.48001 50.6136) (width 0.25) (layer F.Cu) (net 20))
 (segment (start 240.48001 50.6136) (end 240.48001 74.47999) (width 0.25) (layer F.Cu) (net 20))
 (segment (start 209.55 40.64) (end 211.270009 38.919991) (width 0.25) (layer F.Cu) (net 20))
 (segment (start 209.55 41.91) (end 209.55 40.64) (width 0.25) (layer F.Cu) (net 20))
 (segment (start 211.639991 38.919991) (end 228.786401 38.919991) (width 0.25) (layer F.Cu) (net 20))
 (segment (start 211.270009 38.919991) (end 211.639991 38.919991) (width 0.25) (layer F.Cu) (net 20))
 (segment (start 234.31641 80.01) (end 220.98 80.01) (width 0.25) (layer F.Cu) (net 22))
 (segment (start 237.345001 82.009999) (end 236.760001 81.424999) (width 0.25) (layer F.Cu) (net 22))
 (segment (start 235.731409 81.424999) (end 234.31641 80.01) (width 0.25) (layer F.Cu) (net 22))
 (segment (start 236.760001 83.675001) (end 237.345001 83.090001) (width 0.25) (layer F.Cu) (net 22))
 (segment (start 212.578591 83.675001) (end 236.760001 83.675001) (width 0.25) (layer F.Cu) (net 22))
 (segment (start 210.038591 81.135001) (end 212.578591 83.675001) (width 0.25) (layer F.Cu) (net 22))
 (segment (start 193.769999 81.135001) (end 210.038591 81.135001) (width 0.25) (layer F.Cu) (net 22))
 (segment (start 236.760001 81.424999) (end 235.731409 81.424999) (width 0.25) (layer F.Cu) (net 22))
 (segment (start 192.73499 80.099992) (end 193.769999 81.135001) (width 0.25) (layer F.Cu) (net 22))
 (segment (start 192.73499 76.50501) (end 192.73499 80.099992) (width 0.25) (layer F.Cu) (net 22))
 (segment (start 194.31 74.93) (end 192.73499 76.50501) (width 0.25) (layer F.Cu) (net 22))
 (segment (start 237.345001 82.405001) (end 237.345001 82.009999) (width 0.25) (layer F.Cu) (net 22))
 (segment (start 237.345001 82.694999) (end 237.345001 82.405001) (width 0.25) (layer F.Cu) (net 22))
 (segment (start 237.345001 83.090001) (end 237.345001 82.694999) (width 0.25) (layer F.Cu) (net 22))
 (segment (start 241.3 78.74) (end 237.345001 82.694999) (width 0.25) (layer F.Cu) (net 22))
 (segment (start 240.930019 50.430019) (end 241.3 50.8) (width 0.25) (layer F.Cu) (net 22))
 (segment (start 240.930019 50.427199) (end 240.930019 50.430019) (width 0.25) (layer F.Cu) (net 22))
 (segment (start 228.972802 38.469982) (end 240.930019 50.427199) (width 0.25) (layer F.Cu) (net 22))
 (segment (start 206.245016 38.469982) (end 228.972802 38.469982) (width 0.25) (layer F.Cu) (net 22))
 (segment (start 205.74 43.18) (end 205.74 38.974998) (width 0.25) (layer F.Cu) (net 22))
 (segment (start 207.01 44.45) (end 205.74 43.18) (width 0.25) (layer F.Cu) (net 22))
 (segment (start 205.74 38.974998) (end 206.245016 38.469982) (width 0.25) (layer F.Cu) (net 22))
 (segment (start 209.55 44.45) (end 207.01 44.45) (width 0.25) (layer F.Cu) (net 22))
 (segment (start 241.3 50.8) (end 241.3 78.74) (width 0.25) (layer F.Cu) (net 22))
 (segment (start 212.09 41.91) (end 209.55 44.45) (width 0.25) (layer F.Cu) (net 22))
 (segment (start 231.532182 85.09) (end 236.22 85.09) (width 0.25) (layer F.Cu) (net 23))
 (segment (start 227.577183 89.044999) (end 231.532182 85.09) (width 0.25) (layer F.Cu) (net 23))
 (segment (start 210.675001 89.044999) (end 227.577183 89.044999) (width 0.25) (layer F.Cu) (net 23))
 (segment (start 209.55 90.17) (end 210.675001 89.044999) (width 0.25) (layer F.Cu) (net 23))
 (segment (start 220.584998 91.44) (end 225.818592 91.44) (width 0.25) (layer F.Cu) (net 25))
 (segment (start 225.818592 91.44) (end 229.628592 87.63) (width 0.25) (layer F.Cu) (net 25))
 (segment (start 219.314998 92.71) (end 220.584998 91.44) (width 0.25) (layer F.Cu) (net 25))
 (segment (start 229.628592 87.63) (end 236.22 87.63) (width 0.25) (layer F.Cu) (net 25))
 (segment (start 209.55 92.71) (end 219.314998 92.71) (width 0.25) (layer F.Cu) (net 25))
 (segment (start 190.04999 71.57001) (end 190.5 71.12) (width 0.25) (layer F.Cu) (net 28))
 (segment (start 190.04999 79.954992) (end 190.04999 71.57001) (width 0.25) (layer F.Cu) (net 28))
 (segment (start 190.5 80.405002) (end 190.04999 79.954992) (width 0.25) (layer F.Cu) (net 28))
 (segment (start 190.5 83.82) (end 190.5 80.405002) (width 0.25) (layer F.Cu) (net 28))
 (segment (start 193.184999 86.504999) (end 190.5 83.82) (width 0.25) (layer F.Cu) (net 28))
 (segment (start 219.565001 86.504999) (end 193.184999 86.504999) (width 0.25) (layer F.Cu) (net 28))
 (segment (start 220.98 85.09) (end 219.565001 86.504999) (width 0.25) (layer F.Cu) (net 28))
 (segment (start 222.25 41.91) (end 219.71 44.45) (width 0.25) (layer F.Cu) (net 28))
 (segment (start 219.71 44.45) (end 212.09 44.45) (width 0.25) (layer F.Cu) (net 28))
 (segment (start 212.09 44.45) (end 211.45641 44.45) (width 0.25) (layer F.Cu) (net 28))
 (segment (start 211.45641 44.45) (end 207.64641 48.26) (width 0.25) (layer F.Cu) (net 28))
 (segment (start 204.074998 48.26) (end 195.58 56.754998) (width 0.25) (layer F.Cu) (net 28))
 (segment (start 207.64641 48.26) (end 204.074998 48.26) (width 0.25) (layer F.Cu) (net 28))
 (segment (start 195.58 56.754998) (end 195.58 57.15) (width 0.25) (layer F.Cu) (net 28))
 (segment (start 190.5 71.12) (end 194.31 67.31) (width 0.25) (layer F.Cu) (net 28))
 (via (at 190.5 71.12) (size 0.8) (drill 0.4) (layers F.Cu B.Cu) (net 28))
 (via (at 195.58 57.15) (size 0.8) (drill 0.4) (layers F.Cu B.Cu) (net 28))
 (segment (start 190.5 71.12) (end 190.5 58.42) (width 0.25) (layer B.Cu) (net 28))
 (segment (start 191.77 57.15) (end 195.58 57.15) (width 0.25) (layer B.Cu) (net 28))
 (segment (start 190.5 58.42) (end 191.77 57.15) (width 0.25) (layer B.Cu) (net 28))
 (segment (start 194.31 49.53) (end 194.31 58.024998) (width 0.25) (layer F.Cu) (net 30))
 (segment (start 196.85 46.99) (end 194.31 49.53) (width 0.25) (layer F.Cu) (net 30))
 (segment (start 208.28 46.99) (end 196.85 46.99) (width 0.25) (layer F.Cu) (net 30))
 (segment (start 212.09 43.18) (end 208.28 46.99) (width 0.25) (layer F.Cu) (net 30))
 (segment (start 194.31 58.024998) (end 194.31 62.23) (width 0.25) (layer F.Cu) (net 30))
 (segment (start 218.44 43.18) (end 212.09 43.18) (width 0.25) (layer F.Cu) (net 30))
 (segment (start 219.71 41.91) (end 218.44 43.18) (width 0.25) (layer F.Cu) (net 30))
 (segment (start 220.98 82.55) (end 215.9 82.55) (width 0.25) (layer F.Cu) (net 30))
 (segment (start 215.9 82.55) (end 215.9 82.55) (width 0.25) (layer F.Cu) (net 30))
 (via (at 215.9 82.55) (size 0.8) (drill 0.4) (layers F.Cu B.Cu) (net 30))
 (segment (start 194.31 62.23) (end 194.31 64.77) (width 0.25) (layer F.Cu) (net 30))
 (via (at 194.31 62.23) (size 0.8) (drill 0.4) (layers F.Cu B.Cu) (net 30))
 (segment (start 201.93 81.28) (end 201.93 66.04) (width 0.25) (layer B.Cu) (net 30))
 (segment (start 204.47 83.82) (end 201.93 81.28) (width 0.25) (layer B.Cu) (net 30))
 (segment (start 214.63 83.82) (end 204.47 83.82) (width 0.25) (layer B.Cu) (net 30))
 (segment (start 215.9 82.55) (end 214.63 83.82) (width 0.25) (layer B.Cu) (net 30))
 (segment (start 201.93 66.04) (end 198.12 62.23) (width 0.25) (layer B.Cu) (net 30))
 (segment (start 198.12 62.23) (end 194.31 62.23) (width 0.25) (layer B.Cu) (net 30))
 (segment (start 228.6 39.37) (end 237.49 48.26) (width 0.25) (layer F.Cu) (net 34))
 (segment (start 237.49 48.26) (end 237.79501 48.56501) (width 0.25) (layer F.Cu) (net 34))
 (segment (start 237.79501 73.35499) (end 236.22 74.93) (width 0.25) (layer F.Cu) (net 34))
 (segment (start 240.03 71.12) (end 237.79501 73.35499) (width 0.25) (layer F.Cu) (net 34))
 (segment (start 240.03 50.8) (end 240.03 71.12) (width 0.25) (layer F.Cu) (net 34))
 (segment (start 237.49 48.26) (end 240.03 50.8) (width 0.25) (layer F.Cu) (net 34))
 (segment (start 207.01 41.91) (end 208.28 43.18) (width 0.25) (layer F.Cu) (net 34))
 (segment (start 209.945002 43.18) (end 210.82 42.305002) (width 0.25) (layer F.Cu) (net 34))
 (segment (start 209.55 43.18) (end 209.945002 43.18) (width 0.25) (layer F.Cu) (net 34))
 (segment (start 208.28 43.18) (end 209.55 43.18) (width 0.25) (layer F.Cu) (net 34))
 (segment (start 210.82 42.305002) (end 210.82 41.91) (width 0.25) (layer F.Cu) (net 34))
 (segment (start 210.82 41.91) (end 210.82 40.64) (width 0.25) (layer F.Cu) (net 34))
 (segment (start 210.82 40.64) (end 212.09 39.37) (width 0.25) (layer F.Cu) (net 34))
 (segment (start 212.09 39.37) (end 228.6 39.37) (width 0.25) (layer F.Cu) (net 34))
 (segment (start 220.98 62.23) (end 220.98 59.69) (width 0.25) (layer F.Cu) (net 37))
 (segment (start 217.17 55.88) (end 217.17 49.53) (width 0.25) (layer F.Cu) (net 37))
 (segment (start 220.98 59.69) (end 217.17 55.88) (width 0.25) (layer F.Cu) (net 37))
 (segment (start 220.835001 48.115001) (end 214.63 41.91) (width 0.25) (layer B.Cu) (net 35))
 (segment (start 234.409999 63.355001) (end 220.835001 49.780003) (width 0.25) (layer B.Cu) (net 35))
 (segment (start 236.470003 63.355001) (end 234.409999 63.355001) (width 0.25) (layer B.Cu) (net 35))
 (segment (start 237.345001 64.229999) (end 236.470003 63.355001) (width 0.25) (layer B.Cu) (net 35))
 (segment (start 220.835001 49.780003) (end 220.835001 48.115001) (width 0.25) (layer B.Cu) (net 35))
 (segment (start 237.345001 78.884999) (end 237.345001 64.229999) (width 0.25) (layer B.Cu) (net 35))
 (segment (start 236.22 80.01) (end 237.345001 78.884999) (width 0.25) (layer B.Cu) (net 35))
 (segment (start 216.350009 47.809991) (end 214.63 49.53) (width 0.25) (layer F.Cu) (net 31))
 (segment (start 217.17 46.99) (end 216.350009 47.809991) (width 0.25) (layer F.Cu) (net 31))
 (segment (start 227.33 46.99) (end 217.17 46.99) (width 0.25) (layer F.Cu) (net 31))
 (segment (start 237.49 57.15) (end 227.33 46.99) (width 0.25) (layer F.Cu) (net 31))
 (segment (start 237.49 66.04) (end 237.49 57.15) (width 0.25) (layer F.Cu) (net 31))
 (segment (start 236.22 67.31) (end 237.49 66.04) (width 0.25) (layer F.Cu) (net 31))
 (segment (start 238.76 69.85) (end 236.22 72.39) (width 0.25) (layer F.Cu) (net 33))
 (segment (start 239.57999 69.03001) (end 238.76 69.85) (width 0.25) (layer F.Cu) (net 33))
 (segment (start 239.57999 51.61999) (end 239.57999 69.03001) (width 0.25) (layer F.Cu) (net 33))
 (segment (start 228.6 40.64) (end 239.57999 51.61999) (width 0.25) (layer F.Cu) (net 33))
 (segment (start 219.314998 40.64) (end 228.6 40.64) (width 0.25) (layer F.Cu) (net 33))
 (segment (start 218.044998 41.91) (end 219.314998 40.64) (width 0.25) (layer F.Cu) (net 33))
 (segment (start 217.17 41.91) (end 218.044998 41.91) (width 0.25) (layer F.Cu) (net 33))
 (segment (start 207.01 50.8) (end 207.01 49.53) (width 0.25) (layer F.Cu) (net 36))
 (segment (start 220.98 64.77) (end 207.01 50.8) (width 0.25) (layer F.Cu) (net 36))
 (segment (start 238.30999 67.76001) (end 236.22 69.85) (width 0.25) (layer F.Cu) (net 32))
 (segment (start 238.76 55.88) (end 238.76 67.31) (width 0.25) (layer F.Cu) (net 32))
 (segment (start 238.76 67.31) (end 238.30999 67.76001) (width 0.25) (layer F.Cu) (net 32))
 (segment (start 224.79 41.91) (end 238.76 55.88) (width 0.25) (layer F.Cu) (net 32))
 (segment (start 224.934999 73.515001) (end 236.22 62.23) (width 0.25) (layer F.Cu) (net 9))
 (segment (start 210.675001 73.515001) (end 224.934999 73.515001) (width 0.25) (layer F.Cu) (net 9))
 (segment (start 209.55 72.39) (end 210.675001 73.515001) (width 0.25) (layer F.Cu) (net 9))
 (segment (start 236.22 58.42) (end 227.33 49.53) (width 0.25) (layer F.Cu) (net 9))
 (segment (start 236.22 62.23) (end 236.22 58.42) (width 0.25) (layer F.Cu) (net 9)))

